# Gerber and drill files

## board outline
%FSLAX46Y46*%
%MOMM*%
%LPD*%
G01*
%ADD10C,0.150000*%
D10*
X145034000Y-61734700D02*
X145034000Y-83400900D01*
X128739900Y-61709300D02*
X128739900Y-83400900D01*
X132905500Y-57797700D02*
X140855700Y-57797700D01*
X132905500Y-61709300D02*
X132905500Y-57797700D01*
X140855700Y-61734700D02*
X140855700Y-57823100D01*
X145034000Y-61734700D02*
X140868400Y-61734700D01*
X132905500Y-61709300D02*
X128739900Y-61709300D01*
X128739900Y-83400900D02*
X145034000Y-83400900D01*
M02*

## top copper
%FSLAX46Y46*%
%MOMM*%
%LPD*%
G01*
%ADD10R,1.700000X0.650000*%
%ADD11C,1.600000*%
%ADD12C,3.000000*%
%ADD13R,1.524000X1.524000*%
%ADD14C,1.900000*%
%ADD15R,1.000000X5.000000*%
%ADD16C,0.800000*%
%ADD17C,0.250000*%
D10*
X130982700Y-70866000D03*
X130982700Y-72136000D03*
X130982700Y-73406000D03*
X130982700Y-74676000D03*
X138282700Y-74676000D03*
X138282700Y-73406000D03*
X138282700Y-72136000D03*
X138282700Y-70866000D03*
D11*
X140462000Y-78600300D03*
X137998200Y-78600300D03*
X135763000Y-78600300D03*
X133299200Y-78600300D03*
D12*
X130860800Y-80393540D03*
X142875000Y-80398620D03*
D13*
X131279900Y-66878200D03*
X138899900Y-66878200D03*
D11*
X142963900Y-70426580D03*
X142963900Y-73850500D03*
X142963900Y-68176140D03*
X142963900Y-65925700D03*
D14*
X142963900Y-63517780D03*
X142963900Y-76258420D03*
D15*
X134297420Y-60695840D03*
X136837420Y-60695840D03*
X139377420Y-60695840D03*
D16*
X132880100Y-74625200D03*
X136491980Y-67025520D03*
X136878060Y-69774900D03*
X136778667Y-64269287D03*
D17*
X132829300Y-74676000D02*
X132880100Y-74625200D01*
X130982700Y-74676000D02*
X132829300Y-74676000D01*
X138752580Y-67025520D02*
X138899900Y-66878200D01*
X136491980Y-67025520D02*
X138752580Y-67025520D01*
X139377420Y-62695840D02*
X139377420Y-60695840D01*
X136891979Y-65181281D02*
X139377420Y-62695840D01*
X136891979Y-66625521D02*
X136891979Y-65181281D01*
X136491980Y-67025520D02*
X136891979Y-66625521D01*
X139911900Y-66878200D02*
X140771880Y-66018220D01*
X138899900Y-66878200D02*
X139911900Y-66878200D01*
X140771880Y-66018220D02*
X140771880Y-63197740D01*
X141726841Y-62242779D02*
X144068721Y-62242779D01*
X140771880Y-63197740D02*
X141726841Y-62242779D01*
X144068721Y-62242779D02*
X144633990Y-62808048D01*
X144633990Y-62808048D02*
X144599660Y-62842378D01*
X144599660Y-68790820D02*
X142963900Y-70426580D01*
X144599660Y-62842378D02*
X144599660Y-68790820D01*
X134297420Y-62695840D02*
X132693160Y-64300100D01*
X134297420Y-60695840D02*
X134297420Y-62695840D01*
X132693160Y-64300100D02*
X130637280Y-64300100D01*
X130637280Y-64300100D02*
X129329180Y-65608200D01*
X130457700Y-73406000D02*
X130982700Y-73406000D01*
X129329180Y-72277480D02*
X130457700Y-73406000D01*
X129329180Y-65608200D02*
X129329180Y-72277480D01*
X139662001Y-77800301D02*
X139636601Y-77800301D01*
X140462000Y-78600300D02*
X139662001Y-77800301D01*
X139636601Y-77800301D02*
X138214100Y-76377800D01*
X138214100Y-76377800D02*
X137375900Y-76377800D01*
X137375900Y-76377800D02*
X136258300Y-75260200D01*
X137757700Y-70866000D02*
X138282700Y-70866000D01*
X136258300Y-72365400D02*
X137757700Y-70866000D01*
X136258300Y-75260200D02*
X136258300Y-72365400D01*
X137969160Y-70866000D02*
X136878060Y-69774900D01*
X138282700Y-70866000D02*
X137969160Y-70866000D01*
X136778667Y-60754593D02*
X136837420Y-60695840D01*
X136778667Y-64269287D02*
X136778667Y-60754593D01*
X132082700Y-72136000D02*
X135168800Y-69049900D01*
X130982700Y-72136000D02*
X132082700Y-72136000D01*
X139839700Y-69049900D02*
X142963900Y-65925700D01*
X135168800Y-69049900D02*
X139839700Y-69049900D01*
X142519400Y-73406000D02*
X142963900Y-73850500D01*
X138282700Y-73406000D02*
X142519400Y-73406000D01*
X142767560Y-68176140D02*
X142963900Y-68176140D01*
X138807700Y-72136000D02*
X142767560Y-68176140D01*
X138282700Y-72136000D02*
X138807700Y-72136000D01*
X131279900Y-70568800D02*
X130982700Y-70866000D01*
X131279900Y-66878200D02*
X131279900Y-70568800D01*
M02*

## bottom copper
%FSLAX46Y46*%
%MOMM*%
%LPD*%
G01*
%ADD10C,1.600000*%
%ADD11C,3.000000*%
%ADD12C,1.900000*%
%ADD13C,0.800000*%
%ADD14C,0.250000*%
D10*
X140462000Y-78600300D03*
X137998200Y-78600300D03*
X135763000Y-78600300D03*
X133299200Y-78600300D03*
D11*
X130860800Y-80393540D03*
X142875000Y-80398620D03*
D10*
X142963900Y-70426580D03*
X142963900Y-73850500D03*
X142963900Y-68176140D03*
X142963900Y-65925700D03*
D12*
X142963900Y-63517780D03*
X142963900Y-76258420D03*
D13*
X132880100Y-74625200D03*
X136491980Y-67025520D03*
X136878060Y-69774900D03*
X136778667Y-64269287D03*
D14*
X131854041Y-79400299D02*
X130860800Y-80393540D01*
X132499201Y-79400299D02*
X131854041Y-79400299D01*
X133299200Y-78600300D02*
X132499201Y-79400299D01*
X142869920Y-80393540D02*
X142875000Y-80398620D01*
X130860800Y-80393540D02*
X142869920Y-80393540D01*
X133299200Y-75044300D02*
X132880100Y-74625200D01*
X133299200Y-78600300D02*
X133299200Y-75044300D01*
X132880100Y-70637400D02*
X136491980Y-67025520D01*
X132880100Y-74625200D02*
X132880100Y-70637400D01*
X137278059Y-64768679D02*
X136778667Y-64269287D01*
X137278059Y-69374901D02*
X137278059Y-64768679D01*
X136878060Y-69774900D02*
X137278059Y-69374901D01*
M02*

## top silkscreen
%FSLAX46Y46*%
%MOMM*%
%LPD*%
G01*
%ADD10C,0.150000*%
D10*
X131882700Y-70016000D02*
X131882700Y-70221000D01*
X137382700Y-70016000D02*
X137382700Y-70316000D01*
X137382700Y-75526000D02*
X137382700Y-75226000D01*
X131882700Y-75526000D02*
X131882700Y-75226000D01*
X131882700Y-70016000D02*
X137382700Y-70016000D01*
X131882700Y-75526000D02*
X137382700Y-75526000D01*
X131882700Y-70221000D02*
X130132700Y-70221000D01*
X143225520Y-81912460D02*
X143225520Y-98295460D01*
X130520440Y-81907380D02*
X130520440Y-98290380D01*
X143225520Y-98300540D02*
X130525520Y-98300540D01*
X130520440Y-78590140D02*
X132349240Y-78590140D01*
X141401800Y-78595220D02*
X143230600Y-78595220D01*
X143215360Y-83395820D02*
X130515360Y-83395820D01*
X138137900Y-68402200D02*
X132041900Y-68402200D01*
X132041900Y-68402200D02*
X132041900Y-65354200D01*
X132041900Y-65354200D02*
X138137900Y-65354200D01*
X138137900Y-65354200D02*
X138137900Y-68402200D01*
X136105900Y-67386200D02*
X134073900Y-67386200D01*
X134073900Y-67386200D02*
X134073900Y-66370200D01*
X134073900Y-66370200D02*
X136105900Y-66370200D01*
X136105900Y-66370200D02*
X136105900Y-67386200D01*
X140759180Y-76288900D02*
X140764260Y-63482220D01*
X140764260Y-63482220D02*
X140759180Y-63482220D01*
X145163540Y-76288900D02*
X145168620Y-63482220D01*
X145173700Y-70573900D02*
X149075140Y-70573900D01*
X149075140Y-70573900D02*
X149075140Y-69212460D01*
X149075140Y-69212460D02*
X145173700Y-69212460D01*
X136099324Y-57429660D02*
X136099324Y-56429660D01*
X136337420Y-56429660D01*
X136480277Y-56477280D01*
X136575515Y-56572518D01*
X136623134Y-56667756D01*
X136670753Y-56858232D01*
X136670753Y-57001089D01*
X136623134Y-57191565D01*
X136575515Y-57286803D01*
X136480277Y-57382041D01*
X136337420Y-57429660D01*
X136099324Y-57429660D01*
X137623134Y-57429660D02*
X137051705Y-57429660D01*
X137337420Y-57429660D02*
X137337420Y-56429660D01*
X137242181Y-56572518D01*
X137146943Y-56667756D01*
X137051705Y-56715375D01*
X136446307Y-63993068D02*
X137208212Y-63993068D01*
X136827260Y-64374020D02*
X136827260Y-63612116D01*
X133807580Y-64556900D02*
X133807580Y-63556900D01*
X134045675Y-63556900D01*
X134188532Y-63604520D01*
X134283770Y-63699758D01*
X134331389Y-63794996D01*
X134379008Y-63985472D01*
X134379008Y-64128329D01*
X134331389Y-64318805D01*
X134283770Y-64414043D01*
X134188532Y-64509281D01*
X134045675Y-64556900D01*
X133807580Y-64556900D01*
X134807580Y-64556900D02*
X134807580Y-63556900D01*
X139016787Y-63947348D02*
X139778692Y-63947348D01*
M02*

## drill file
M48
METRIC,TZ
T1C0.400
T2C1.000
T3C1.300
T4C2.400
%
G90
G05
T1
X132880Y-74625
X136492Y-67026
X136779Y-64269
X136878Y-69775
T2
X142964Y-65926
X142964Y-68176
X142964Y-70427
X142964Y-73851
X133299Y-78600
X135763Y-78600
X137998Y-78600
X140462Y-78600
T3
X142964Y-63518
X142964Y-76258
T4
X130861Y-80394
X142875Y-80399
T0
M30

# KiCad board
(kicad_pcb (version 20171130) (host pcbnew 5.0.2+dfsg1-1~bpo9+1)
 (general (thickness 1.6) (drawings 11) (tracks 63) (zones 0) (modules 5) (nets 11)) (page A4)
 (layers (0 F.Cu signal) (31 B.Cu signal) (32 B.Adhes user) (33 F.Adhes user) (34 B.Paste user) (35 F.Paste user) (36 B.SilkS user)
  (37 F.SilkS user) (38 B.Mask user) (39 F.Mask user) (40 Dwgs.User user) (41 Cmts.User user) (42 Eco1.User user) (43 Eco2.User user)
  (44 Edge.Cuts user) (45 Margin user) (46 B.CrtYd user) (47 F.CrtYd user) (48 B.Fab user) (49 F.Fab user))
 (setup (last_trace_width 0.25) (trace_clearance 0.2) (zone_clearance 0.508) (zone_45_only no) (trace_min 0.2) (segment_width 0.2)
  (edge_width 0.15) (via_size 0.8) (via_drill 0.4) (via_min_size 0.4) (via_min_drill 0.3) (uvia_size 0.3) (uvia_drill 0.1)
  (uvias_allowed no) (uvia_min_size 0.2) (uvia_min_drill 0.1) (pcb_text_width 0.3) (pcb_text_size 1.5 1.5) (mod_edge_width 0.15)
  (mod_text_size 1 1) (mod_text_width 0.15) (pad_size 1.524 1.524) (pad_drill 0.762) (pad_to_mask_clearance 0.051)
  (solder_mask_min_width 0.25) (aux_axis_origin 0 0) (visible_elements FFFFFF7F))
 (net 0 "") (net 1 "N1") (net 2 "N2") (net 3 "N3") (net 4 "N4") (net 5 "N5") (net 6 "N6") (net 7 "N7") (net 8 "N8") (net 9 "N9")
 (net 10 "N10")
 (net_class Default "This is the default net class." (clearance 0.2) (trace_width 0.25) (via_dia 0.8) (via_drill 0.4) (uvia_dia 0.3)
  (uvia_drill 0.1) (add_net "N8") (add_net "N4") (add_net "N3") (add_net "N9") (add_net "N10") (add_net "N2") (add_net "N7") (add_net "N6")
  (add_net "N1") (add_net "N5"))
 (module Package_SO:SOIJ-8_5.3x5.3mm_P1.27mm (layer F.Cu) (at 134.6327 72.771)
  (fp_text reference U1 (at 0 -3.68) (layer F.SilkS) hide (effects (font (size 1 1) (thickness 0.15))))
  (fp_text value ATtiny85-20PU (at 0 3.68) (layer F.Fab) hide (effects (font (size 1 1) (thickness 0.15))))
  (fp_line (start -2.75 -2.755) (end -2.75 -2.55) (layer F.SilkS) (width 0.15))
  (fp_line (start 2.75 -2.755) (end 2.75 -2.455) (layer F.SilkS) (width 0.15))
  (fp_line (start 2.75 2.755) (end 2.75 2.455) (layer F.SilkS) (width 0.15))
  (fp_line (start -2.75 2.755) (end -2.75 2.455) (layer F.SilkS) (width 0.15))
  (fp_line (start -2.75 -2.755) (end 2.75 -2.755) (layer F.SilkS) (width 0.15))
  (fp_line (start -2.75 2.755) (end 2.75 2.755) (layer F.SilkS) (width 0.15))
  (fp_line (start -2.75 -2.55) (end -4.5 -2.55) (layer F.SilkS) (width 0.15))
  (pad 1 smd rect (at -3.65 -1.905) (size 1.7 0.65) (layers F.Cu F.Paste F.Mask) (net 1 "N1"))
  (pad 2 smd rect (at -3.65 -0.635) (size 1.7 0.65) (layers F.Cu F.Paste F.Mask) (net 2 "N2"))
  (pad 3 smd rect (at -3.65 0.635) (size 1.7 0.65) (layers F.Cu F.Paste F.Mask) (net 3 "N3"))
  (pad 4 smd rect (at -3.65 1.905) (size 1.7 0.65) (layers F.Cu F.Paste F.Mask) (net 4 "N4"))
  (pad 5 smd rect (at 3.65 1.905) (size 1.7 0.65) (layers F.Cu F.Paste F.Mask) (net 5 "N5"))
  (pad 6 smd rect (at 3.65 0.635) (size 1.7 0.65) (layers F.Cu F.Paste F.Mask) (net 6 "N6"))
  (pad 7 smd rect (at 3.65 -0.635) (size 1.7 0.65) (layers F.Cu F.Paste F.Mask) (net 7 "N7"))
  (pad 8 smd rect (at 3.65 -1.905) (size 1.7 0.65) (layers F.Cu F.Paste F.Mask) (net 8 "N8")))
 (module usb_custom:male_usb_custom (layer F.Cu) (at 136.8806 78.6003 180)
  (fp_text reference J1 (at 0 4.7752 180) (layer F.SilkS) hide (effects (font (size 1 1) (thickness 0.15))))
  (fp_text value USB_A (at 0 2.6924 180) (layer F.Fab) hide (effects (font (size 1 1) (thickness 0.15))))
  (fp_line (start -6.34492 -3.31216) (end -6.34492 -19.69516) (layer F.SilkS) (width 0.15))
  (fp_line (start 6.36016 -3.30708) (end 6.36016 -19.69008) (layer F.SilkS) (width 0.15))
  (fp_line (start -6.34492 -19.70024) (end 6.35508 -19.70024) (layer F.SilkS) (width 0.15))
  (fp_line (start 6.36016 0.01016) (end 4.53136 0.01016) (layer F.SilkS) (width 0.15))
  (fp_line (start -4.5212 0.00508) (end -6.35 0.00508) (layer F.SilkS) (width 0.15))
  (fp_line (start -6.33476 -4.79552) (end 6.36524 -4.79552) (layer F.SilkS) (width 0.15))
  (pad 1 thru_hole circle (at -3.5814 0 180) (size 1.6 1.6) (drill 1) (layers *.Cu *.Mask) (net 8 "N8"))
  (pad 2 thru_hole circle (at -1.1176 0 180) (size 1.6 1.6) (drill 1) (layers *.Cu *.Mask) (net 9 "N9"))
  (pad 3 thru_hole circle (at 1.1176 0 180) (size 1.6 1.6) (drill 1) (layers *.Cu *.Mask) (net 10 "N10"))
  (pad 4 thru_hole circle (at 3.5814 0 180) (size 1.6 1.6) (drill 1) (layers *.Cu *.Mask) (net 4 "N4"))
  (pad 4 thru_hole circle (at 6.0198 -1.79324 180) (size 3 3) (drill 2.4) (layers *.Cu *.Mask) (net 4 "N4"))
  (pad 4 thru_hole circle (at -5.9944 -1.79832 180) (size 3 3) (drill 2.4) (layers *.Cu *.Mask) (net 4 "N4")))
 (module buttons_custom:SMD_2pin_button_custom (layer F.Cu) (at 135.0899 66.8782 180)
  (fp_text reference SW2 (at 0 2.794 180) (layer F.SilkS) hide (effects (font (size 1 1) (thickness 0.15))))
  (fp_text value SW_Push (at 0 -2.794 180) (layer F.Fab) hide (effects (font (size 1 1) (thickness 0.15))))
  (fp_line (start -3.048 -1.524) (end 3.048 -1.524) (layer F.SilkS) (width 0.15))
  (fp_line (start 3.048 -1.524) (end 3.048 1.524) (layer F.SilkS) (width 0.15))
  (fp_line (start 3.048 1.524) (end -3.048 1.524) (layer F.SilkS) (width 0.15))
  (fp_line (start -3.048 1.524) (end -3.048 -1.524) (layer F.SilkS) (width 0.15))
  (fp_line (start -1.016 -0.508) (end 1.016 -0.508) (layer F.SilkS) (width 0.15))
  (fp_line (start 1.016 -0.508) (end 1.016 0.508) (layer F.SilkS) (width 0.15))
  (fp_line (start 1.016 0.508) (end -1.016 0.508) (layer F.SilkS) (width 0.15))
  (fp_line (start -1.016 0.508) (end -1.016 -0.508) (layer F.SilkS) (width 0.15))
  (pad 1 smd rect (at 3.81 0 180) (size 1.524 1.524) (layers F.Cu F.Paste F.Mask) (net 1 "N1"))
  (pad 2 smd rect (at -3.81 0 180) (size 1.524 1.524) (layers F.Cu F.Paste F.Mask) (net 4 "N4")))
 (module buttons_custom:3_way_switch (layer F.Cu) (at 142.9639 69.8881 90)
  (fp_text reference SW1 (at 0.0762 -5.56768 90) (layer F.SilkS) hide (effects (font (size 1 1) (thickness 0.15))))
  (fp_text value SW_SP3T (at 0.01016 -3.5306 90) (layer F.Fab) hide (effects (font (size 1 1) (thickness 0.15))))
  (fp_line (start -6.4008 -2.20472) (end 6.40588 -2.19964) (layer F.SilkS) (width 0.15))
  (fp_line (start 6.40588 -2.19964) (end 6.40588 -2.20472) (layer F.SilkS) (width 0.15))
  (fp_line (start -6.4008 2.19964) (end 6.40588 2.20472) (layer F.SilkS) (width 0.15))
  (fp_line (start -0.6858 2.2098) (end -0.6858 6.11124) (layer F.SilkS) (width 0.15))
  (fp_line (start -0.6858 6.11124) (end 0.67564 6.11124) (layer F.SilkS) (width 0.15))
  (fp_line (start 0.67564 6.11124) (end 0.67564 2.2098) (layer F.SilkS) (width 0.15))
  (pad 3 thru_hole circle (at -0.53848 0 90) (size 1.6 1.6) (drill 1) (layers *.Cu *.Mask) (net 4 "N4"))
  (pad 4 thru_hole circle (at -3.9624 0 90) (size 1.6 1.6) (drill 1) (layers *.Cu *.Mask) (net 6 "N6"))
  (pad 2 thru_hole circle (at 1.71196 0 90) (size 1.6 1.6) (drill 1) (layers *.Cu *.Mask) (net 7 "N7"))
  (pad 1 thru_hole circle (at 3.9624 0 90) (size 1.6 1.6) (drill 1) (layers *.Cu *.Mask) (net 2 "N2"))
  (pad 5 thru_hole circle (at 6.37032 0 90) (size 1.9 1.9) (drill 1.3) (layers *.Cu *.Mask))
  (pad 6 thru_hole circle (at -6.37032 0 90) (size 1.9 1.9) (drill 1.3) (layers *.Cu *.Mask)))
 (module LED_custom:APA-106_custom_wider (layer F.Cu) (at 136.83742 60.69584)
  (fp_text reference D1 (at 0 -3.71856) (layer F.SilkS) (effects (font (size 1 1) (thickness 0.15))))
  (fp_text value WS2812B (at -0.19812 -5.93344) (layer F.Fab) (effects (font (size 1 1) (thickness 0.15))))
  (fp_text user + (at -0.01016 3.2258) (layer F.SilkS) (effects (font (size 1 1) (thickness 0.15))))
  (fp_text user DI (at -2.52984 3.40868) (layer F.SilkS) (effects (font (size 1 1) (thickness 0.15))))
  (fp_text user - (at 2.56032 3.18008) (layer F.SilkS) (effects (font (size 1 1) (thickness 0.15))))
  (pad 4 smd rect (at -2.54 0) (size 1 5) (layers F.Cu F.Paste F.Mask) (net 3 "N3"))
  (pad 1 smd rect (at 0 0) (size 1 5) (layers F.Cu F.Paste F.Mask) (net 8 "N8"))
  (pad 3 smd rect (at 2.54 0) (size 1 5) (layers F.Cu F.Paste F.Mask) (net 4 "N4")))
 (gr_line (start 145.034 61.7347) (end 145.034 83.4009) (layer Edge.Cuts) (width 0.15))
 (gr_line (start 128.7399 61.7093) (end 128.7399 83.4009) (layer Edge.Cuts) (width 0.15))
 (gr_line (start 132.9055 57.7977) (end 140.8557 57.7977) (layer Edge.Cuts) (width 0.15))
 (gr_line (start 132.9055 61.7093) (end 132.9055 57.7977) (layer Edge.Cuts) (width 0.15))
 (gr_line (start 140.8557 61.7347) (end 140.8557 57.8231) (layer Edge.Cuts) (width 0.15))
 (gr_line (start 145.034 61.7347) (end 140.8684 61.7347) (layer Edge.Cuts) (width 0.15))
 (gr_line (start 132.9055 61.7093) (end 128.7399 61.7093) (layer Edge.Cuts) (width 0.15))
 (gr_line (start 128.7399 83.4009) (end 145.034 83.4009) (layer Edge.Cuts) (width 0.15))
 (segment (start 132.8293 74.676) (end 132.8801 74.6252) (width 0.25) (layer F.Cu) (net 4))
 (via (at 132.8801 74.6252) (size 0.8) (drill 0.4) (layers F.Cu B.Cu) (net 4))
 (segment (start 130.9827 74.676) (end 132.8293 74.676) (width 0.25) (layer F.Cu) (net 4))
 (segment (start 131.854041 79.400299) (end 130.8608 80.39354) (width 0.25) (layer B.Cu) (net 4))
 (segment (start 132.499201 79.400299) (end 131.854041 79.400299) (width 0.25) (layer B.Cu) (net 4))
 (segment (start 133.2992 78.6003) (end 132.499201 79.400299) (width 0.25) (layer B.Cu) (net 4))
 (segment (start 142.86992 80.39354) (end 142.875 80.39862) (width 0.25) (layer B.Cu) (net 4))
 (segment (start 130.8608 80.39354) (end 142.86992 80.39354) (width 0.25) (layer B.Cu) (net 4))
 (segment (start 133.2992 75.0443) (end 132.8801 74.6252) (width 0.25) (layer B.Cu) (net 4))
 (segment (start 133.2992 78.6003) (end 133.2992 75.0443) (width 0.25) (layer B.Cu) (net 4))
 (via (at 136.49198 67.02552) (size 0.8) (drill 0.4) (layers F.Cu B.Cu) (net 4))
 (segment (start 132.8801 70.6374) (end 136.49198 67.02552) (width 0.25) (layer B.Cu) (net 4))
 (segment (start 132.8801 74.6252) (end 132.8801 70.6374) (width 0.25) (layer B.Cu) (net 4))
 (segment (start 138.75258 67.02552) (end 138.8999 66.8782) (width 0.25) (layer F.Cu) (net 4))
 (segment (start 136.49198 67.02552) (end 138.75258 67.02552) (width 0.25) (layer F.Cu) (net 4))
 (segment (start 139.37742 62.69584) (end 139.37742 60.69584) (width 0.25) (layer F.Cu) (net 4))
 (segment (start 136.891979 65.181281) (end 139.37742 62.69584) (width 0.25) (layer F.Cu) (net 4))
 (segment (start 136.891979 66.625521) (end 136.891979 65.181281) (width 0.25) (layer F.Cu) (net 4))
 (segment (start 136.49198 67.02552) (end 136.891979 66.625521) (width 0.25) (layer F.Cu) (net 4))
 (segment (start 139.9119 66.8782) (end 140.77188 66.01822) (width 0.25) (layer F.Cu) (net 4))
 (segment (start 138.8999 66.8782) (end 139.9119 66.8782) (width 0.25) (layer F.Cu) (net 4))
 (segment (start 140.77188 66.01822) (end 140.77188 63.19774) (width 0.25) (layer F.Cu) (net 4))
 (segment (start 141.726841 62.242779) (end 144.068721 62.242779) (width 0.25) (layer F.Cu) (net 4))
 (segment (start 140.77188 63.19774) (end 141.726841 62.242779) (width 0.25) (layer F.Cu) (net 4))
 (segment (start 144.068721 62.242779) (end 144.63399 62.808048) (width 0.25) (layer F.Cu) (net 4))
 (segment (start 144.63399 62.808048) (end 144.59966 62.842378) (width 0.25) (layer F.Cu) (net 4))
 (segment (start 144.59966 68.79082) (end 142.9639 70.42658) (width 0.25) (layer F.Cu) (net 4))
 (segment (start 144.59966 62.842378) (end 144.59966 68.79082) (width 0.25) (layer F.Cu) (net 4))
 (segment (start 134.29742 62.69584) (end 132.69316 64.3001) (width 0.25) (layer F.Cu) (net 3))
 (segment (start 134.29742 60.69584) (end 134.29742 62.69584) (width 0.25) (layer F.Cu) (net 3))
 (segment (start 132.69316 64.3001) (end 130.63728 64.3001) (width 0.25) (layer F.Cu) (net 3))
 (segment (start 130.63728 64.3001) (end 129.32918 65.6082) (width 0.25) (layer F.Cu) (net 3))
 (segment (start 130.4577 73.406) (end 130.9827 73.406) (width 0.25) (layer F.Cu) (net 3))
 (segment (start 129.32918 72.27748) (end 130.4577 73.406) (width 0.25) (layer F.Cu) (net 3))
 (segment (start 129.32918 65.6082) (end 129.32918 72.27748) (width 0.25) (layer F.Cu) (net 3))
 (segment (start 139.662001 77.800301) (end 139.636601 77.800301) (width 0.25) (layer F.Cu) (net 8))
 (segment (start 140.462 78.6003) (end 139.662001 77.800301) (width 0.25) (layer F.Cu) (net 8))
 (segment (start 139.636601 77.800301) (end 138.2141 76.3778) (width 0.25) (layer F.Cu) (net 8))
 (segment (start 138.2141 76.3778) (end 137.3759 76.3778) (width 0.25) (layer F.Cu) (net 8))
 (segment (start 137.3759 76.3778) (end 136.2583 75.2602) (width 0.25) (layer F.Cu) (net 8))
 (segment (start 137.7577 70.866) (end 138.2827 70.866) (width 0.25) (layer F.Cu) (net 8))
 (segment (start 136.2583 72.3654) (end 137.7577 70.866) (width 0.25) (layer F.Cu) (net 8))
 (segment (start 136.2583 75.2602) (end 136.2583 72.3654) (width 0.25) (layer F.Cu) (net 8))
 (via (at 136.87806 69.7749) (size 0.8) (drill 0.4) (layers F.Cu B.Cu) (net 8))
 (segment (start 137.96916 70.866) (end 136.87806 69.7749) (width 0.25) (layer F.Cu) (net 8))
 (segment (start 138.2827 70.866) (end 137.96916 70.866) (width 0.25) (layer F.Cu) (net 8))
 (via (at 136.778667 64.269287) (size 0.8) (drill 0.4) (layers F.Cu B.Cu) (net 8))
 (segment (start 137.278059 64.768679) (end 136.778667 64.269287) (width 0.25) (layer B.Cu) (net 8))
 (segment (start 137.278059 69.374901) (end 137.278059 64.768679) (width 0.25) (layer B.Cu) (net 8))
 (segment (start 136.87806 69.7749) (end 137.278059 69.374901) (width 0.25) (layer B.Cu) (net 8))
 (segment (start 136.778667 60.754593) (end 136.83742 60.69584) (width 0.25) (layer F.Cu) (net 8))
 (segment (start 136.778667 64.269287) (end 136.778667 60.754593) (width 0.25) (layer F.Cu) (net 8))
 (segment (start 132.0827 72.136) (end 135.1688 69.0499) (width 0.25) (layer F.Cu) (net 2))
 (segment (start 130.9827 72.136) (end 132.0827 72.136) (width 0.25) (layer F.Cu) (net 2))
 (segment (start 139.8397 69.0499) (end 142.9639 65.9257) (width 0.25) (layer F.Cu) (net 2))
 (segment (start 135.1688 69.0499) (end 139.8397 69.0499) (width 0.25) (layer F.Cu) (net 2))
 (segment (start 142.5194 73.406) (end 142.9639 73.8505) (width 0.25) (layer F.Cu) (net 6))
 (segment (start 138.2827 73.406) (end 142.5194 73.406) (width 0.25) (layer F.Cu) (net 6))
 (segment (start 142.76756 68.17614) (end 142.9639 68.17614) (width 0.25) (layer F.Cu) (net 7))
 (segment (start 138.8077 72.136) (end 142.76756 68.17614) (width 0.25) (layer F.Cu) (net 7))
 (segment (start 138.2827 72.136) (end 138.8077 72.136) (width 0.25) (layer F.Cu) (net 7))
 (segment (start 131.2799 70.5688) (end 130.9827 70.866) (width 0.25) (layer F.Cu) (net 1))
 (segment (start 131.2799 66.8782) (end 131.2799 70.5688) (width 0.25) (layer F.Cu) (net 1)))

